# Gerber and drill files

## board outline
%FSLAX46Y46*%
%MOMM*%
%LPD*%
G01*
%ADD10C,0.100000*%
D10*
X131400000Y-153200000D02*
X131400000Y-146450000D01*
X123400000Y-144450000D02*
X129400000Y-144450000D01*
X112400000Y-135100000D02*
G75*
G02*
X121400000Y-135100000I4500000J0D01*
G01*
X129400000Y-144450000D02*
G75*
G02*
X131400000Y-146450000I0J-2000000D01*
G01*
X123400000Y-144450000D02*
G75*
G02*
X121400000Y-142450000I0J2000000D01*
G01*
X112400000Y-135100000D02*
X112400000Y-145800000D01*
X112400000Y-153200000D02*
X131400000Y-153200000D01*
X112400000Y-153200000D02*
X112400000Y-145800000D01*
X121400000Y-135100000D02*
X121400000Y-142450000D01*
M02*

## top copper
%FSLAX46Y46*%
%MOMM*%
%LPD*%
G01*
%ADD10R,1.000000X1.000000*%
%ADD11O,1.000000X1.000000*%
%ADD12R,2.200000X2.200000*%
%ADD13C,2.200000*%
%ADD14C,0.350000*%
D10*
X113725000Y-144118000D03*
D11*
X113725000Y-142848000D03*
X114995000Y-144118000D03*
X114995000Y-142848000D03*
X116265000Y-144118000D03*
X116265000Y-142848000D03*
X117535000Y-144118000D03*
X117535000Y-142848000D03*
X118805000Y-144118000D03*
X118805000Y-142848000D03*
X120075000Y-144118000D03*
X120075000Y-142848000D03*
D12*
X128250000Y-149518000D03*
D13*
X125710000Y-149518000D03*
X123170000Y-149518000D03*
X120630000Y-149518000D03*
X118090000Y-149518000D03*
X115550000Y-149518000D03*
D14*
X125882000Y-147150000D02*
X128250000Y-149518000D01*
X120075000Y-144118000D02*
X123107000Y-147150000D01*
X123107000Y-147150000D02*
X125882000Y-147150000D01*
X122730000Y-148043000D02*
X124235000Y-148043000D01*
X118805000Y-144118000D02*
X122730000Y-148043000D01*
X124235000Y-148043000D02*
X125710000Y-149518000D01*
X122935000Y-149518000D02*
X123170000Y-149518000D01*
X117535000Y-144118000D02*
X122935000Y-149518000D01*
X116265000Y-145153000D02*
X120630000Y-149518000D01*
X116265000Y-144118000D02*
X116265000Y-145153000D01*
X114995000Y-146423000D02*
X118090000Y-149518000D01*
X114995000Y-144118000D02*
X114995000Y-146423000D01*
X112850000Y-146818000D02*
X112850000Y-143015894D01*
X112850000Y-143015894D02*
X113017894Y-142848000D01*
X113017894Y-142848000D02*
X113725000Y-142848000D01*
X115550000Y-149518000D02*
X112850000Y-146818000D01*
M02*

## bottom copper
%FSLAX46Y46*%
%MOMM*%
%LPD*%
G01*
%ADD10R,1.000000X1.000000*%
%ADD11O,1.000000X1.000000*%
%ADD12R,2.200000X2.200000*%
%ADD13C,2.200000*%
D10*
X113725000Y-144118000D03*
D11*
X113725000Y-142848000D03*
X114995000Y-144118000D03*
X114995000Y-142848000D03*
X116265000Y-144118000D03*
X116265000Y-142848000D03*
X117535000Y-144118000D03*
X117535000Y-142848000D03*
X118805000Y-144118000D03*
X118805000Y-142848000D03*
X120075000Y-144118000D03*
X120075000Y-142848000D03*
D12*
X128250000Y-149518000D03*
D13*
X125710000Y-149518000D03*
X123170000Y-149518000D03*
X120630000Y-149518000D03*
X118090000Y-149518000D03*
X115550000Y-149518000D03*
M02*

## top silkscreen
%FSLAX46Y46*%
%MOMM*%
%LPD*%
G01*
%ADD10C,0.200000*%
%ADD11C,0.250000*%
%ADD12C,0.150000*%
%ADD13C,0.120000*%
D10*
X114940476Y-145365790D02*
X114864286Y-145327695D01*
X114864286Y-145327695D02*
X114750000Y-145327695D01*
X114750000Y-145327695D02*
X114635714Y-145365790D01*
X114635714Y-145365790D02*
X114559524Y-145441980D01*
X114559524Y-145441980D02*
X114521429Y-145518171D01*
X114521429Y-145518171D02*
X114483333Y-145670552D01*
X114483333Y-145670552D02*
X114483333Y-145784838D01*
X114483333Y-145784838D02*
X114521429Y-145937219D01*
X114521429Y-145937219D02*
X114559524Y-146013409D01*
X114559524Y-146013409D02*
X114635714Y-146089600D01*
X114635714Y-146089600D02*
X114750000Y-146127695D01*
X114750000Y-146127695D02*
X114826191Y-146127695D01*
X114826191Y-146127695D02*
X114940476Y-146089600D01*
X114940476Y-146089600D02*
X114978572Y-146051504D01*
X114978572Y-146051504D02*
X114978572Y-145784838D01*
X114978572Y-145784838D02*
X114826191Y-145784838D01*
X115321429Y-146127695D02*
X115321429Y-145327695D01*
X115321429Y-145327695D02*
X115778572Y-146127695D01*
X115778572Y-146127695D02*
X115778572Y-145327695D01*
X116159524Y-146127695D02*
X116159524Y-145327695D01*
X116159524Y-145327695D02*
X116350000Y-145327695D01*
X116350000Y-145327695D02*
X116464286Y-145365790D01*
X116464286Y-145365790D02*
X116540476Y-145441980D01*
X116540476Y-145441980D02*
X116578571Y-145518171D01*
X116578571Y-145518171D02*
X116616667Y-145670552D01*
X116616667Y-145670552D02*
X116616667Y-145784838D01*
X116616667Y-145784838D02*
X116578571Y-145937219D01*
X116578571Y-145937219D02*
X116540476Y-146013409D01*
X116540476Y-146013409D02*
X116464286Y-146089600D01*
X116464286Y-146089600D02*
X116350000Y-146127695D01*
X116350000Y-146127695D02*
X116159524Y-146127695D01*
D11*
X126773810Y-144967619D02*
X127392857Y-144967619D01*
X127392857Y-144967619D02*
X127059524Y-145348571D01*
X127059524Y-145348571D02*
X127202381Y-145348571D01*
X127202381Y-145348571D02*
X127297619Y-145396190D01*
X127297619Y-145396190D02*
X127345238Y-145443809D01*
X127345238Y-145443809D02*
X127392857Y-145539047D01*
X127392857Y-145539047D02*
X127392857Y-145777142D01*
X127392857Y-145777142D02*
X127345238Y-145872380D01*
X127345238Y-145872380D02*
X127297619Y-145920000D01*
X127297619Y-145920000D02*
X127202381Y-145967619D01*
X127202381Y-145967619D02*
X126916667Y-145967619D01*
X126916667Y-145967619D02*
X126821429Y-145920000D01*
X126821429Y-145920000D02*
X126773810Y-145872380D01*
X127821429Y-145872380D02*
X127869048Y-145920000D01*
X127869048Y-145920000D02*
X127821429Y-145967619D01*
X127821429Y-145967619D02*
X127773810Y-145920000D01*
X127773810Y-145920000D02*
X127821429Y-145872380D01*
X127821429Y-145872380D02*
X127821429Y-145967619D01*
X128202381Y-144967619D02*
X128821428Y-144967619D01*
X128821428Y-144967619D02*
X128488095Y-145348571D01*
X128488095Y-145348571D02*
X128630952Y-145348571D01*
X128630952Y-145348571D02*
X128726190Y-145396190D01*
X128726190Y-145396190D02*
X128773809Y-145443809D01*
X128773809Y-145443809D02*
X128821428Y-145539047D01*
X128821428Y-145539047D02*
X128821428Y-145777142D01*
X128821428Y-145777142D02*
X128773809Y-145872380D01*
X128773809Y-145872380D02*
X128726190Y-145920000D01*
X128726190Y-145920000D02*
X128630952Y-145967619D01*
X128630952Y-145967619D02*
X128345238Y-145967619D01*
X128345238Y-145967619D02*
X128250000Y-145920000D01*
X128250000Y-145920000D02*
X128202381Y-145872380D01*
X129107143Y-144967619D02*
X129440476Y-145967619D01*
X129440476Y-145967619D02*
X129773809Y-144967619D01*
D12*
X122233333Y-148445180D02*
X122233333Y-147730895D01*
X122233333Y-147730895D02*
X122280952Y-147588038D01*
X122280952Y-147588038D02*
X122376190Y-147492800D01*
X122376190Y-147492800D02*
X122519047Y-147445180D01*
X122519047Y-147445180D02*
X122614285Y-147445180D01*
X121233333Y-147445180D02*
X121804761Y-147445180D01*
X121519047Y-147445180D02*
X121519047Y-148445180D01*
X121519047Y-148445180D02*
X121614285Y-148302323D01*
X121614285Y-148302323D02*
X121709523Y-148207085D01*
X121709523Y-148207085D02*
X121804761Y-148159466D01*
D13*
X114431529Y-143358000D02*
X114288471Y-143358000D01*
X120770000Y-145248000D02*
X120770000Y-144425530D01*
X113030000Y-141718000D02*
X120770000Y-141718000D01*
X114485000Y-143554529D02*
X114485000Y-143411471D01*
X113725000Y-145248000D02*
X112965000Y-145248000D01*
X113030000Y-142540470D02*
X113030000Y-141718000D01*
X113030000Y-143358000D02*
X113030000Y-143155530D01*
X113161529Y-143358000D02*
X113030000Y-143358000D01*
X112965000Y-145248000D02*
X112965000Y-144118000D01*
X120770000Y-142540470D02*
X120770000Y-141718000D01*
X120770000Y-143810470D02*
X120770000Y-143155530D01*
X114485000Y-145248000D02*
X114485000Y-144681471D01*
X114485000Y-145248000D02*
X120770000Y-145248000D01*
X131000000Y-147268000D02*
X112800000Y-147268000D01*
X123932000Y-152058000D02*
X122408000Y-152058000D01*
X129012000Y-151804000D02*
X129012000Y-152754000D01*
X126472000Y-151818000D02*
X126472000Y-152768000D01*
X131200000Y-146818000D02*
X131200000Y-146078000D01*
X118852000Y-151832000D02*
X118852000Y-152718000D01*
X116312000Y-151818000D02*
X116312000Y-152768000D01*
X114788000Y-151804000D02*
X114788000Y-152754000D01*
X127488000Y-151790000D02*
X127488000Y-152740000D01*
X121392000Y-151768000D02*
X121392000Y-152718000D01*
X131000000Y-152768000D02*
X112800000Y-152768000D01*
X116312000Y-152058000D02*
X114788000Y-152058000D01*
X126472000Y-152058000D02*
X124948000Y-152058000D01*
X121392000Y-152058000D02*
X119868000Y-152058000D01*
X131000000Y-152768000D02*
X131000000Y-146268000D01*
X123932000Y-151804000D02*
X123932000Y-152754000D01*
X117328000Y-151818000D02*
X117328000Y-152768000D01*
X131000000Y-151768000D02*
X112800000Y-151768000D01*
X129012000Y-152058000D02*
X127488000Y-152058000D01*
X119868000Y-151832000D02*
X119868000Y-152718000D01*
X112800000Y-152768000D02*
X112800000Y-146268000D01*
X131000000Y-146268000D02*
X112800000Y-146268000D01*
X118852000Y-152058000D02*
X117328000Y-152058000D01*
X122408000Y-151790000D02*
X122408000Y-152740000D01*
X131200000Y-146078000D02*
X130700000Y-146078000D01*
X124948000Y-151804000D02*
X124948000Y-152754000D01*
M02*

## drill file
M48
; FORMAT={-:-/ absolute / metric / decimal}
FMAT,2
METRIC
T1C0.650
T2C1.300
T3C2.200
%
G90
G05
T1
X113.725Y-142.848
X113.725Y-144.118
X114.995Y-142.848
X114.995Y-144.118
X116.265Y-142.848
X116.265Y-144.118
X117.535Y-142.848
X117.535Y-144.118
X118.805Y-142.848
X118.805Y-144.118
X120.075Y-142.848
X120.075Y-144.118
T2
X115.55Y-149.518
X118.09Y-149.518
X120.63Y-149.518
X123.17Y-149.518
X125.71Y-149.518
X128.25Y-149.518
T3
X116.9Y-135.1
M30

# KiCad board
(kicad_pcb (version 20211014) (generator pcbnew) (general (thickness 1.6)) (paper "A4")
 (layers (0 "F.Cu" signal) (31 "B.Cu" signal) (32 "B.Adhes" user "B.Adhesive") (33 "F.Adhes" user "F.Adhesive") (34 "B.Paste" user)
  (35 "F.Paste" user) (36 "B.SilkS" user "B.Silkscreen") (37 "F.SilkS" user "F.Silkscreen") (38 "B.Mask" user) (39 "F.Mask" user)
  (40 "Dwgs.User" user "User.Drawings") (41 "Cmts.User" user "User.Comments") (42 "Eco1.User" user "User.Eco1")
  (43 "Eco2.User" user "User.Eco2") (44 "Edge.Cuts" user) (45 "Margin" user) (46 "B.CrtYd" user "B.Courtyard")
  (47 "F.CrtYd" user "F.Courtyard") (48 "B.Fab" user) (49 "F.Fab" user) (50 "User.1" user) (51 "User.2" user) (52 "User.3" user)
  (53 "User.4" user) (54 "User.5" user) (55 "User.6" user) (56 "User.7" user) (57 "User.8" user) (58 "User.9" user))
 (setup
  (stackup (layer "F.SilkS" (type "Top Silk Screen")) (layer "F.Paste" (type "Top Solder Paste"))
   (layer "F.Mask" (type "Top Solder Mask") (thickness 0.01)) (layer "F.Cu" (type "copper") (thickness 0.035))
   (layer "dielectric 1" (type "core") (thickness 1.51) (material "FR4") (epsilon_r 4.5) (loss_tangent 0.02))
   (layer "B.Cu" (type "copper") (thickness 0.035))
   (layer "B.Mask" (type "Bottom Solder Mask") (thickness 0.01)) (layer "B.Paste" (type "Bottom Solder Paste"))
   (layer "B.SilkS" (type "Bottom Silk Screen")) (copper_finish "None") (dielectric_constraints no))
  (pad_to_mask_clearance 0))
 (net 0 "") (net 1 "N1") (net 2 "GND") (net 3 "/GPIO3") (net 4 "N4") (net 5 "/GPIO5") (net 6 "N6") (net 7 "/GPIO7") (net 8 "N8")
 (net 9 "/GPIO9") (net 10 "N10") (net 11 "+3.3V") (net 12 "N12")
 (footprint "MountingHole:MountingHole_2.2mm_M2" (layer "F.Cu") (at 116.9 135.1)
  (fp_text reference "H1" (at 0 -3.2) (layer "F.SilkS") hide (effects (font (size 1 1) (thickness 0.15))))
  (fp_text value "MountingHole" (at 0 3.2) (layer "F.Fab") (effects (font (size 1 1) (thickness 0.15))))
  (pad "" np_thru_hole circle (at 0 0) (size 2.2 2.2) (drill 2.2) (layers *.Cu *.Mask)))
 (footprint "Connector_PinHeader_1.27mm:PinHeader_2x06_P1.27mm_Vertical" (layer "F.Cu") (at 113.725 144.118 90)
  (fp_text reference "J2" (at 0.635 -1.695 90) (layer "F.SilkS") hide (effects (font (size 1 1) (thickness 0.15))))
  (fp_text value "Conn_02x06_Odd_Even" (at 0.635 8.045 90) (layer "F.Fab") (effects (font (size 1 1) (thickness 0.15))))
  (fp_line (start 0.76 0.706529) (end 0.76 0.563471) (layer "F.SilkS") (width 0.12))
  (fp_line (start -1.13 7.045) (end -0.30753 7.045) (layer "F.SilkS") (width 0.12))
  (fp_line (start 2.4 -0.695) (end 2.4 7.045) (layer "F.SilkS") (width 0.12))
  (fp_line (start 0.563471 0.76) (end 0.706529 0.76) (layer "F.SilkS") (width 0.12))
  (fp_line (start -1.13 0) (end -1.13 -0.76) (layer "F.SilkS") (width 0.12))
  (fp_line (start 1.57753 -0.695) (end 2.4 -0.695) (layer "F.SilkS") (width 0.12))
  (fp_line (start 0.76 -0.695) (end 0.96247 -0.695) (layer "F.SilkS") (width 0.12))
  (fp_line (start 0.76 -0.563471) (end 0.76 -0.695) (layer "F.SilkS") (width 0.12))
  (fp_line (start -1.13 -0.76) (end 0 -0.76) (layer "F.SilkS") (width 0.12))
  (fp_line (start 1.57753 7.045) (end 2.4 7.045) (layer "F.SilkS") (width 0.12))
  (fp_line (start 0.30753 7.045) (end 0.96247 7.045) (layer "F.SilkS") (width 0.12))
  (fp_line (start -1.13 0.76) (end -0.563471 0.76) (layer "F.SilkS") (width 0.12))
  (fp_line (start -1.13 0.76) (end -1.13 7.045) (layer "F.SilkS") (width 0.12))
  (pad "1" thru_hole rect (at 0 0 90) (size 1 1) (drill 0.65) (layers *.Cu *.Mask) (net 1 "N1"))
  (pad "2" thru_hole oval (at 1.27 0 90) (size 1 1) (drill 0.65) (layers *.Cu *.Mask) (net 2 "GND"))
  (pad "3" thru_hole oval (at 0 1.27 90) (size 1 1) (drill 0.65) (layers *.Cu *.Mask) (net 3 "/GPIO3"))
  (pad "4" thru_hole oval (at 1.27 1.27 90) (size 1 1) (drill 0.65) (layers *.Cu *.Mask) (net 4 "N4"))
  (pad "5" thru_hole oval (at 0 2.54 90) (size 1 1) (drill 0.65) (layers *.Cu *.Mask) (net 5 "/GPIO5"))
  (pad "6" thru_hole oval (at 1.27 2.54 90) (size 1 1) (drill 0.65) (layers *.Cu *.Mask) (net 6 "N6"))
  (pad "7" thru_hole oval (at 0 3.81 90) (size 1 1) (drill 0.65) (layers *.Cu *.Mask) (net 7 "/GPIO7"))
  (pad "8" thru_hole oval (at 1.27 3.81 90) (size 1 1) (drill 0.65) (layers *.Cu *.Mask) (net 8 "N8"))
  (pad "9" thru_hole oval (at 0 5.08 90) (size 1 1) (drill 0.65) (layers *.Cu *.Mask) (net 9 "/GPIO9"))
  (pad "10" thru_hole oval (at 1.27 5.08 90) (size 1 1) (drill 0.65) (layers *.Cu *.Mask) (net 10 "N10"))
  (pad "11" thru_hole oval (at 0 6.35 90) (size 1 1) (drill 0.65) (layers *.Cu *.Mask) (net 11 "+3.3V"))
  (pad "12" thru_hole oval (at 1.27 6.35 90) (size 1 1) (drill 0.65) (layers *.Cu *.Mask) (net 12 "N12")))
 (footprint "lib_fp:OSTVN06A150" (layer "F.Cu") (at 121.9 149.518 180)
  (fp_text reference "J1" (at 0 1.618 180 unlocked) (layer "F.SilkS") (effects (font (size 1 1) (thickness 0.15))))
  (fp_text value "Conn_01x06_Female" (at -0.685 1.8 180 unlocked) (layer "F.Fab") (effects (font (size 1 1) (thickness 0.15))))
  (fp_line (start -9.1 2.25) (end 9.1 2.25) (layer "F.SilkS") (width 0.12))
  (fp_line (start -2.032 -2.54) (end -0.508 -2.54) (layer "F.SilkS") (width 0.12))
  (fp_line (start -7.112 -2.286) (end -7.112 -3.236) (layer "F.SilkS") (width 0.12))
  (fp_line (start -4.572 -2.3) (end -4.572 -3.25) (layer "F.SilkS") (width 0.12))
  (fp_line (start -9.3 2.7) (end -9.3 3.44) (layer "F.SilkS") (width 0.12))
  (fp_line (start 3.048 -2.314) (end 3.048 -3.2) (layer "F.SilkS") (width 0.12))
  (fp_line (start 5.588 -2.3) (end 5.588 -3.25) (layer "F.SilkS") (width 0.12))
  (fp_line (start 7.112 -2.286) (end 7.112 -3.236) (layer "F.SilkS") (width 0.12))
  (fp_line (start -5.588 -2.272) (end -5.588 -3.222) (layer "F.SilkS") (width 0.12))
  (fp_line (start 0.508 -2.25) (end 0.508 -3.2) (layer "F.SilkS") (width 0.12))
  (fp_line (start -9.1 -3.25) (end 9.1 -3.25) (layer "F.SilkS") (width 0.12))
  (fp_line (start 5.588 -2.54) (end 7.112 -2.54) (layer "F.SilkS") (width 0.12))
  (fp_line (start -4.572 -2.54) (end -3.048 -2.54) (layer "F.SilkS") (width 0.12))
  (fp_line (start 0.508 -2.54) (end 2.032 -2.54) (layer "F.SilkS") (width 0.12))
  (fp_line (start -9.1 -3.25) (end -9.1 3.25) (layer "F.SilkS") (width 0.12))
  (fp_line (start -2.032 -2.286) (end -2.032 -3.236) (layer "F.SilkS") (width 0.12))
  (fp_line (start 4.572 -2.3) (end 4.572 -3.25) (layer "F.SilkS") (width 0.12))
  (fp_line (start -9.1 -2.25) (end 9.1 -2.25) (layer "F.SilkS") (width 0.12))
  (fp_line (start -7.112 -2.54) (end -5.588 -2.54) (layer "F.SilkS") (width 0.12))
  (fp_line (start 2.032 -2.314) (end 2.032 -3.2) (layer "F.SilkS") (width 0.12))
  (fp_line (start 9.1 -3.25) (end 9.1 3.25) (layer "F.SilkS") (width 0.12))
  (fp_line (start -9.1 3.25) (end 9.1 3.25) (layer "F.SilkS") (width 0.12))
  (fp_line (start 3.048 -2.54) (end 4.572 -2.54) (layer "F.SilkS") (width 0.12))
  (fp_line (start -0.508 -2.272) (end -0.508 -3.222) (layer "F.SilkS") (width 0.12))
  (fp_line (start -9.3 3.44) (end -8.8 3.44) (layer "F.SilkS") (width 0.12))
  (fp_line (start -3.048 -2.286) (end -3.048 -3.236) (layer "F.SilkS") (width 0.12))
  (pad "1" thru_hole rect (at -6.35 0 180) (size 2.2 2.2) (drill 1.3) (layers *.Cu *.Mask) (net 11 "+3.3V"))
  (pad "2" thru_hole circle (at -3.81 0 180) (size 2.2 2.2) (drill 1.3) (layers *.Cu *.Mask) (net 9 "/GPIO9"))
  (pad "3" thru_hole circle (at -1.27 0 180) (size 2.2 2.2) (drill 1.3) (layers *.Cu *.Mask) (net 7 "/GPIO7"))
  (pad "4" thru_hole circle (at 1.27 0 180) (size 2.2 2.2) (drill 1.3) (layers *.Cu *.Mask) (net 5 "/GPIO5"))
  (pad "5" thru_hole circle (at 3.81 0 180) (size 2.2 2.2) (drill 1.3) (layers *.Cu *.Mask) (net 3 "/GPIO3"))
  (pad "6" thru_hole circle (at 6.35 0 180) (size 2.2 2.2) (drill 1.3) (layers *.Cu *.Mask) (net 2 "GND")))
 (gr_line (start 131.4 153.2) (end 131.4 146.45) (layer "Edge.Cuts") (width 0.1))
 (gr_line (start 123.4 144.45) (end 129.4 144.45) (layer "Edge.Cuts") (width 0.1))
 (gr_arc (start 112.4 135.1) (mid 116.9 130.6) (end 121.4 135.1) (layer "Edge.Cuts") (width 0.1))
 (gr_arc (start 129.4 144.45) (mid 130.814213 145.035787) (end 131.4 146.45) (layer "Edge.Cuts") (width 0.1))
 (gr_arc (start 123.4 144.45) (mid 121.985786 143.864213) (end 121.4 142.45) (layer "Edge.Cuts") (width 0.1))
 (gr_line (start 112.4 135.1) (end 112.4 145.8) (layer "Edge.Cuts") (width 0.1))
 (gr_line (start 112.4 153.2) (end 131.4 153.2) (layer "Edge.Cuts") (width 0.1))
 (gr_line (start 112.4 153.2) (end 112.4 145.8) (layer "Edge.Cuts") (width 0.1))
 (gr_line (start 121.4 135.1) (end 121.4 142.45) (layer "Edge.Cuts") (width 0.1))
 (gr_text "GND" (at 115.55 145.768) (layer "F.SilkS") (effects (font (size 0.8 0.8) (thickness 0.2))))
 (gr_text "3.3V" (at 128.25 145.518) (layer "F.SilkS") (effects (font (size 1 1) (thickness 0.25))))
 (segment (start 125.882 147.15) (end 128.25 149.518) (width 0.35) (layer "F.Cu") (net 11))
 (segment (start 120.075 144.118) (end 123.107 147.15) (width 0.35) (layer "F.Cu") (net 11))
 (segment (start 123.107 147.15) (end 125.882 147.15) (width 0.35) (layer "F.Cu") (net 11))
 (segment (start 122.73 148.043) (end 124.235 148.043) (width 0.35) (layer "F.Cu") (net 9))
 (segment (start 118.805 144.118) (end 122.73 148.043) (width 0.35) (layer "F.Cu") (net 9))
 (segment (start 124.235 148.043) (end 125.71 149.518) (width 0.35) (layer "F.Cu") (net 9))
 (segment (start 122.935 149.518) (end 123.17 149.518) (width 0.35) (layer "F.Cu") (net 7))
 (segment (start 117.535 144.118) (end 122.935 149.518) (width 0.35) (layer "F.Cu") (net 7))
 (segment (start 116.265 145.153) (end 120.63 149.518) (width 0.35) (layer "F.Cu") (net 5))
 (segment (start 116.265 144.118) (end 116.265 145.153) (width 0.35) (layer "F.Cu") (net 5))
 (segment (start 114.995 146.423) (end 118.09 149.518) (width 0.35) (layer "F.Cu") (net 3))
 (segment (start 114.995 144.118) (end 114.995 146.423) (width 0.35) (layer "F.Cu") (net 3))
 (segment (start 112.85 146.818) (end 112.85 143.015894) (width 0.35) (layer "F.Cu") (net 2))
 (segment (start 112.85 143.015894) (end 113.017894 142.848) (width 0.35) (layer "F.Cu") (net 2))
 (segment (start 113.017894 142.848) (end 113.725 142.848) (width 0.35) (layer "F.Cu") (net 2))
 (segment (start 115.55 149.518) (end 112.85 146.818) (width 0.35) (layer "F.Cu") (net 2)))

